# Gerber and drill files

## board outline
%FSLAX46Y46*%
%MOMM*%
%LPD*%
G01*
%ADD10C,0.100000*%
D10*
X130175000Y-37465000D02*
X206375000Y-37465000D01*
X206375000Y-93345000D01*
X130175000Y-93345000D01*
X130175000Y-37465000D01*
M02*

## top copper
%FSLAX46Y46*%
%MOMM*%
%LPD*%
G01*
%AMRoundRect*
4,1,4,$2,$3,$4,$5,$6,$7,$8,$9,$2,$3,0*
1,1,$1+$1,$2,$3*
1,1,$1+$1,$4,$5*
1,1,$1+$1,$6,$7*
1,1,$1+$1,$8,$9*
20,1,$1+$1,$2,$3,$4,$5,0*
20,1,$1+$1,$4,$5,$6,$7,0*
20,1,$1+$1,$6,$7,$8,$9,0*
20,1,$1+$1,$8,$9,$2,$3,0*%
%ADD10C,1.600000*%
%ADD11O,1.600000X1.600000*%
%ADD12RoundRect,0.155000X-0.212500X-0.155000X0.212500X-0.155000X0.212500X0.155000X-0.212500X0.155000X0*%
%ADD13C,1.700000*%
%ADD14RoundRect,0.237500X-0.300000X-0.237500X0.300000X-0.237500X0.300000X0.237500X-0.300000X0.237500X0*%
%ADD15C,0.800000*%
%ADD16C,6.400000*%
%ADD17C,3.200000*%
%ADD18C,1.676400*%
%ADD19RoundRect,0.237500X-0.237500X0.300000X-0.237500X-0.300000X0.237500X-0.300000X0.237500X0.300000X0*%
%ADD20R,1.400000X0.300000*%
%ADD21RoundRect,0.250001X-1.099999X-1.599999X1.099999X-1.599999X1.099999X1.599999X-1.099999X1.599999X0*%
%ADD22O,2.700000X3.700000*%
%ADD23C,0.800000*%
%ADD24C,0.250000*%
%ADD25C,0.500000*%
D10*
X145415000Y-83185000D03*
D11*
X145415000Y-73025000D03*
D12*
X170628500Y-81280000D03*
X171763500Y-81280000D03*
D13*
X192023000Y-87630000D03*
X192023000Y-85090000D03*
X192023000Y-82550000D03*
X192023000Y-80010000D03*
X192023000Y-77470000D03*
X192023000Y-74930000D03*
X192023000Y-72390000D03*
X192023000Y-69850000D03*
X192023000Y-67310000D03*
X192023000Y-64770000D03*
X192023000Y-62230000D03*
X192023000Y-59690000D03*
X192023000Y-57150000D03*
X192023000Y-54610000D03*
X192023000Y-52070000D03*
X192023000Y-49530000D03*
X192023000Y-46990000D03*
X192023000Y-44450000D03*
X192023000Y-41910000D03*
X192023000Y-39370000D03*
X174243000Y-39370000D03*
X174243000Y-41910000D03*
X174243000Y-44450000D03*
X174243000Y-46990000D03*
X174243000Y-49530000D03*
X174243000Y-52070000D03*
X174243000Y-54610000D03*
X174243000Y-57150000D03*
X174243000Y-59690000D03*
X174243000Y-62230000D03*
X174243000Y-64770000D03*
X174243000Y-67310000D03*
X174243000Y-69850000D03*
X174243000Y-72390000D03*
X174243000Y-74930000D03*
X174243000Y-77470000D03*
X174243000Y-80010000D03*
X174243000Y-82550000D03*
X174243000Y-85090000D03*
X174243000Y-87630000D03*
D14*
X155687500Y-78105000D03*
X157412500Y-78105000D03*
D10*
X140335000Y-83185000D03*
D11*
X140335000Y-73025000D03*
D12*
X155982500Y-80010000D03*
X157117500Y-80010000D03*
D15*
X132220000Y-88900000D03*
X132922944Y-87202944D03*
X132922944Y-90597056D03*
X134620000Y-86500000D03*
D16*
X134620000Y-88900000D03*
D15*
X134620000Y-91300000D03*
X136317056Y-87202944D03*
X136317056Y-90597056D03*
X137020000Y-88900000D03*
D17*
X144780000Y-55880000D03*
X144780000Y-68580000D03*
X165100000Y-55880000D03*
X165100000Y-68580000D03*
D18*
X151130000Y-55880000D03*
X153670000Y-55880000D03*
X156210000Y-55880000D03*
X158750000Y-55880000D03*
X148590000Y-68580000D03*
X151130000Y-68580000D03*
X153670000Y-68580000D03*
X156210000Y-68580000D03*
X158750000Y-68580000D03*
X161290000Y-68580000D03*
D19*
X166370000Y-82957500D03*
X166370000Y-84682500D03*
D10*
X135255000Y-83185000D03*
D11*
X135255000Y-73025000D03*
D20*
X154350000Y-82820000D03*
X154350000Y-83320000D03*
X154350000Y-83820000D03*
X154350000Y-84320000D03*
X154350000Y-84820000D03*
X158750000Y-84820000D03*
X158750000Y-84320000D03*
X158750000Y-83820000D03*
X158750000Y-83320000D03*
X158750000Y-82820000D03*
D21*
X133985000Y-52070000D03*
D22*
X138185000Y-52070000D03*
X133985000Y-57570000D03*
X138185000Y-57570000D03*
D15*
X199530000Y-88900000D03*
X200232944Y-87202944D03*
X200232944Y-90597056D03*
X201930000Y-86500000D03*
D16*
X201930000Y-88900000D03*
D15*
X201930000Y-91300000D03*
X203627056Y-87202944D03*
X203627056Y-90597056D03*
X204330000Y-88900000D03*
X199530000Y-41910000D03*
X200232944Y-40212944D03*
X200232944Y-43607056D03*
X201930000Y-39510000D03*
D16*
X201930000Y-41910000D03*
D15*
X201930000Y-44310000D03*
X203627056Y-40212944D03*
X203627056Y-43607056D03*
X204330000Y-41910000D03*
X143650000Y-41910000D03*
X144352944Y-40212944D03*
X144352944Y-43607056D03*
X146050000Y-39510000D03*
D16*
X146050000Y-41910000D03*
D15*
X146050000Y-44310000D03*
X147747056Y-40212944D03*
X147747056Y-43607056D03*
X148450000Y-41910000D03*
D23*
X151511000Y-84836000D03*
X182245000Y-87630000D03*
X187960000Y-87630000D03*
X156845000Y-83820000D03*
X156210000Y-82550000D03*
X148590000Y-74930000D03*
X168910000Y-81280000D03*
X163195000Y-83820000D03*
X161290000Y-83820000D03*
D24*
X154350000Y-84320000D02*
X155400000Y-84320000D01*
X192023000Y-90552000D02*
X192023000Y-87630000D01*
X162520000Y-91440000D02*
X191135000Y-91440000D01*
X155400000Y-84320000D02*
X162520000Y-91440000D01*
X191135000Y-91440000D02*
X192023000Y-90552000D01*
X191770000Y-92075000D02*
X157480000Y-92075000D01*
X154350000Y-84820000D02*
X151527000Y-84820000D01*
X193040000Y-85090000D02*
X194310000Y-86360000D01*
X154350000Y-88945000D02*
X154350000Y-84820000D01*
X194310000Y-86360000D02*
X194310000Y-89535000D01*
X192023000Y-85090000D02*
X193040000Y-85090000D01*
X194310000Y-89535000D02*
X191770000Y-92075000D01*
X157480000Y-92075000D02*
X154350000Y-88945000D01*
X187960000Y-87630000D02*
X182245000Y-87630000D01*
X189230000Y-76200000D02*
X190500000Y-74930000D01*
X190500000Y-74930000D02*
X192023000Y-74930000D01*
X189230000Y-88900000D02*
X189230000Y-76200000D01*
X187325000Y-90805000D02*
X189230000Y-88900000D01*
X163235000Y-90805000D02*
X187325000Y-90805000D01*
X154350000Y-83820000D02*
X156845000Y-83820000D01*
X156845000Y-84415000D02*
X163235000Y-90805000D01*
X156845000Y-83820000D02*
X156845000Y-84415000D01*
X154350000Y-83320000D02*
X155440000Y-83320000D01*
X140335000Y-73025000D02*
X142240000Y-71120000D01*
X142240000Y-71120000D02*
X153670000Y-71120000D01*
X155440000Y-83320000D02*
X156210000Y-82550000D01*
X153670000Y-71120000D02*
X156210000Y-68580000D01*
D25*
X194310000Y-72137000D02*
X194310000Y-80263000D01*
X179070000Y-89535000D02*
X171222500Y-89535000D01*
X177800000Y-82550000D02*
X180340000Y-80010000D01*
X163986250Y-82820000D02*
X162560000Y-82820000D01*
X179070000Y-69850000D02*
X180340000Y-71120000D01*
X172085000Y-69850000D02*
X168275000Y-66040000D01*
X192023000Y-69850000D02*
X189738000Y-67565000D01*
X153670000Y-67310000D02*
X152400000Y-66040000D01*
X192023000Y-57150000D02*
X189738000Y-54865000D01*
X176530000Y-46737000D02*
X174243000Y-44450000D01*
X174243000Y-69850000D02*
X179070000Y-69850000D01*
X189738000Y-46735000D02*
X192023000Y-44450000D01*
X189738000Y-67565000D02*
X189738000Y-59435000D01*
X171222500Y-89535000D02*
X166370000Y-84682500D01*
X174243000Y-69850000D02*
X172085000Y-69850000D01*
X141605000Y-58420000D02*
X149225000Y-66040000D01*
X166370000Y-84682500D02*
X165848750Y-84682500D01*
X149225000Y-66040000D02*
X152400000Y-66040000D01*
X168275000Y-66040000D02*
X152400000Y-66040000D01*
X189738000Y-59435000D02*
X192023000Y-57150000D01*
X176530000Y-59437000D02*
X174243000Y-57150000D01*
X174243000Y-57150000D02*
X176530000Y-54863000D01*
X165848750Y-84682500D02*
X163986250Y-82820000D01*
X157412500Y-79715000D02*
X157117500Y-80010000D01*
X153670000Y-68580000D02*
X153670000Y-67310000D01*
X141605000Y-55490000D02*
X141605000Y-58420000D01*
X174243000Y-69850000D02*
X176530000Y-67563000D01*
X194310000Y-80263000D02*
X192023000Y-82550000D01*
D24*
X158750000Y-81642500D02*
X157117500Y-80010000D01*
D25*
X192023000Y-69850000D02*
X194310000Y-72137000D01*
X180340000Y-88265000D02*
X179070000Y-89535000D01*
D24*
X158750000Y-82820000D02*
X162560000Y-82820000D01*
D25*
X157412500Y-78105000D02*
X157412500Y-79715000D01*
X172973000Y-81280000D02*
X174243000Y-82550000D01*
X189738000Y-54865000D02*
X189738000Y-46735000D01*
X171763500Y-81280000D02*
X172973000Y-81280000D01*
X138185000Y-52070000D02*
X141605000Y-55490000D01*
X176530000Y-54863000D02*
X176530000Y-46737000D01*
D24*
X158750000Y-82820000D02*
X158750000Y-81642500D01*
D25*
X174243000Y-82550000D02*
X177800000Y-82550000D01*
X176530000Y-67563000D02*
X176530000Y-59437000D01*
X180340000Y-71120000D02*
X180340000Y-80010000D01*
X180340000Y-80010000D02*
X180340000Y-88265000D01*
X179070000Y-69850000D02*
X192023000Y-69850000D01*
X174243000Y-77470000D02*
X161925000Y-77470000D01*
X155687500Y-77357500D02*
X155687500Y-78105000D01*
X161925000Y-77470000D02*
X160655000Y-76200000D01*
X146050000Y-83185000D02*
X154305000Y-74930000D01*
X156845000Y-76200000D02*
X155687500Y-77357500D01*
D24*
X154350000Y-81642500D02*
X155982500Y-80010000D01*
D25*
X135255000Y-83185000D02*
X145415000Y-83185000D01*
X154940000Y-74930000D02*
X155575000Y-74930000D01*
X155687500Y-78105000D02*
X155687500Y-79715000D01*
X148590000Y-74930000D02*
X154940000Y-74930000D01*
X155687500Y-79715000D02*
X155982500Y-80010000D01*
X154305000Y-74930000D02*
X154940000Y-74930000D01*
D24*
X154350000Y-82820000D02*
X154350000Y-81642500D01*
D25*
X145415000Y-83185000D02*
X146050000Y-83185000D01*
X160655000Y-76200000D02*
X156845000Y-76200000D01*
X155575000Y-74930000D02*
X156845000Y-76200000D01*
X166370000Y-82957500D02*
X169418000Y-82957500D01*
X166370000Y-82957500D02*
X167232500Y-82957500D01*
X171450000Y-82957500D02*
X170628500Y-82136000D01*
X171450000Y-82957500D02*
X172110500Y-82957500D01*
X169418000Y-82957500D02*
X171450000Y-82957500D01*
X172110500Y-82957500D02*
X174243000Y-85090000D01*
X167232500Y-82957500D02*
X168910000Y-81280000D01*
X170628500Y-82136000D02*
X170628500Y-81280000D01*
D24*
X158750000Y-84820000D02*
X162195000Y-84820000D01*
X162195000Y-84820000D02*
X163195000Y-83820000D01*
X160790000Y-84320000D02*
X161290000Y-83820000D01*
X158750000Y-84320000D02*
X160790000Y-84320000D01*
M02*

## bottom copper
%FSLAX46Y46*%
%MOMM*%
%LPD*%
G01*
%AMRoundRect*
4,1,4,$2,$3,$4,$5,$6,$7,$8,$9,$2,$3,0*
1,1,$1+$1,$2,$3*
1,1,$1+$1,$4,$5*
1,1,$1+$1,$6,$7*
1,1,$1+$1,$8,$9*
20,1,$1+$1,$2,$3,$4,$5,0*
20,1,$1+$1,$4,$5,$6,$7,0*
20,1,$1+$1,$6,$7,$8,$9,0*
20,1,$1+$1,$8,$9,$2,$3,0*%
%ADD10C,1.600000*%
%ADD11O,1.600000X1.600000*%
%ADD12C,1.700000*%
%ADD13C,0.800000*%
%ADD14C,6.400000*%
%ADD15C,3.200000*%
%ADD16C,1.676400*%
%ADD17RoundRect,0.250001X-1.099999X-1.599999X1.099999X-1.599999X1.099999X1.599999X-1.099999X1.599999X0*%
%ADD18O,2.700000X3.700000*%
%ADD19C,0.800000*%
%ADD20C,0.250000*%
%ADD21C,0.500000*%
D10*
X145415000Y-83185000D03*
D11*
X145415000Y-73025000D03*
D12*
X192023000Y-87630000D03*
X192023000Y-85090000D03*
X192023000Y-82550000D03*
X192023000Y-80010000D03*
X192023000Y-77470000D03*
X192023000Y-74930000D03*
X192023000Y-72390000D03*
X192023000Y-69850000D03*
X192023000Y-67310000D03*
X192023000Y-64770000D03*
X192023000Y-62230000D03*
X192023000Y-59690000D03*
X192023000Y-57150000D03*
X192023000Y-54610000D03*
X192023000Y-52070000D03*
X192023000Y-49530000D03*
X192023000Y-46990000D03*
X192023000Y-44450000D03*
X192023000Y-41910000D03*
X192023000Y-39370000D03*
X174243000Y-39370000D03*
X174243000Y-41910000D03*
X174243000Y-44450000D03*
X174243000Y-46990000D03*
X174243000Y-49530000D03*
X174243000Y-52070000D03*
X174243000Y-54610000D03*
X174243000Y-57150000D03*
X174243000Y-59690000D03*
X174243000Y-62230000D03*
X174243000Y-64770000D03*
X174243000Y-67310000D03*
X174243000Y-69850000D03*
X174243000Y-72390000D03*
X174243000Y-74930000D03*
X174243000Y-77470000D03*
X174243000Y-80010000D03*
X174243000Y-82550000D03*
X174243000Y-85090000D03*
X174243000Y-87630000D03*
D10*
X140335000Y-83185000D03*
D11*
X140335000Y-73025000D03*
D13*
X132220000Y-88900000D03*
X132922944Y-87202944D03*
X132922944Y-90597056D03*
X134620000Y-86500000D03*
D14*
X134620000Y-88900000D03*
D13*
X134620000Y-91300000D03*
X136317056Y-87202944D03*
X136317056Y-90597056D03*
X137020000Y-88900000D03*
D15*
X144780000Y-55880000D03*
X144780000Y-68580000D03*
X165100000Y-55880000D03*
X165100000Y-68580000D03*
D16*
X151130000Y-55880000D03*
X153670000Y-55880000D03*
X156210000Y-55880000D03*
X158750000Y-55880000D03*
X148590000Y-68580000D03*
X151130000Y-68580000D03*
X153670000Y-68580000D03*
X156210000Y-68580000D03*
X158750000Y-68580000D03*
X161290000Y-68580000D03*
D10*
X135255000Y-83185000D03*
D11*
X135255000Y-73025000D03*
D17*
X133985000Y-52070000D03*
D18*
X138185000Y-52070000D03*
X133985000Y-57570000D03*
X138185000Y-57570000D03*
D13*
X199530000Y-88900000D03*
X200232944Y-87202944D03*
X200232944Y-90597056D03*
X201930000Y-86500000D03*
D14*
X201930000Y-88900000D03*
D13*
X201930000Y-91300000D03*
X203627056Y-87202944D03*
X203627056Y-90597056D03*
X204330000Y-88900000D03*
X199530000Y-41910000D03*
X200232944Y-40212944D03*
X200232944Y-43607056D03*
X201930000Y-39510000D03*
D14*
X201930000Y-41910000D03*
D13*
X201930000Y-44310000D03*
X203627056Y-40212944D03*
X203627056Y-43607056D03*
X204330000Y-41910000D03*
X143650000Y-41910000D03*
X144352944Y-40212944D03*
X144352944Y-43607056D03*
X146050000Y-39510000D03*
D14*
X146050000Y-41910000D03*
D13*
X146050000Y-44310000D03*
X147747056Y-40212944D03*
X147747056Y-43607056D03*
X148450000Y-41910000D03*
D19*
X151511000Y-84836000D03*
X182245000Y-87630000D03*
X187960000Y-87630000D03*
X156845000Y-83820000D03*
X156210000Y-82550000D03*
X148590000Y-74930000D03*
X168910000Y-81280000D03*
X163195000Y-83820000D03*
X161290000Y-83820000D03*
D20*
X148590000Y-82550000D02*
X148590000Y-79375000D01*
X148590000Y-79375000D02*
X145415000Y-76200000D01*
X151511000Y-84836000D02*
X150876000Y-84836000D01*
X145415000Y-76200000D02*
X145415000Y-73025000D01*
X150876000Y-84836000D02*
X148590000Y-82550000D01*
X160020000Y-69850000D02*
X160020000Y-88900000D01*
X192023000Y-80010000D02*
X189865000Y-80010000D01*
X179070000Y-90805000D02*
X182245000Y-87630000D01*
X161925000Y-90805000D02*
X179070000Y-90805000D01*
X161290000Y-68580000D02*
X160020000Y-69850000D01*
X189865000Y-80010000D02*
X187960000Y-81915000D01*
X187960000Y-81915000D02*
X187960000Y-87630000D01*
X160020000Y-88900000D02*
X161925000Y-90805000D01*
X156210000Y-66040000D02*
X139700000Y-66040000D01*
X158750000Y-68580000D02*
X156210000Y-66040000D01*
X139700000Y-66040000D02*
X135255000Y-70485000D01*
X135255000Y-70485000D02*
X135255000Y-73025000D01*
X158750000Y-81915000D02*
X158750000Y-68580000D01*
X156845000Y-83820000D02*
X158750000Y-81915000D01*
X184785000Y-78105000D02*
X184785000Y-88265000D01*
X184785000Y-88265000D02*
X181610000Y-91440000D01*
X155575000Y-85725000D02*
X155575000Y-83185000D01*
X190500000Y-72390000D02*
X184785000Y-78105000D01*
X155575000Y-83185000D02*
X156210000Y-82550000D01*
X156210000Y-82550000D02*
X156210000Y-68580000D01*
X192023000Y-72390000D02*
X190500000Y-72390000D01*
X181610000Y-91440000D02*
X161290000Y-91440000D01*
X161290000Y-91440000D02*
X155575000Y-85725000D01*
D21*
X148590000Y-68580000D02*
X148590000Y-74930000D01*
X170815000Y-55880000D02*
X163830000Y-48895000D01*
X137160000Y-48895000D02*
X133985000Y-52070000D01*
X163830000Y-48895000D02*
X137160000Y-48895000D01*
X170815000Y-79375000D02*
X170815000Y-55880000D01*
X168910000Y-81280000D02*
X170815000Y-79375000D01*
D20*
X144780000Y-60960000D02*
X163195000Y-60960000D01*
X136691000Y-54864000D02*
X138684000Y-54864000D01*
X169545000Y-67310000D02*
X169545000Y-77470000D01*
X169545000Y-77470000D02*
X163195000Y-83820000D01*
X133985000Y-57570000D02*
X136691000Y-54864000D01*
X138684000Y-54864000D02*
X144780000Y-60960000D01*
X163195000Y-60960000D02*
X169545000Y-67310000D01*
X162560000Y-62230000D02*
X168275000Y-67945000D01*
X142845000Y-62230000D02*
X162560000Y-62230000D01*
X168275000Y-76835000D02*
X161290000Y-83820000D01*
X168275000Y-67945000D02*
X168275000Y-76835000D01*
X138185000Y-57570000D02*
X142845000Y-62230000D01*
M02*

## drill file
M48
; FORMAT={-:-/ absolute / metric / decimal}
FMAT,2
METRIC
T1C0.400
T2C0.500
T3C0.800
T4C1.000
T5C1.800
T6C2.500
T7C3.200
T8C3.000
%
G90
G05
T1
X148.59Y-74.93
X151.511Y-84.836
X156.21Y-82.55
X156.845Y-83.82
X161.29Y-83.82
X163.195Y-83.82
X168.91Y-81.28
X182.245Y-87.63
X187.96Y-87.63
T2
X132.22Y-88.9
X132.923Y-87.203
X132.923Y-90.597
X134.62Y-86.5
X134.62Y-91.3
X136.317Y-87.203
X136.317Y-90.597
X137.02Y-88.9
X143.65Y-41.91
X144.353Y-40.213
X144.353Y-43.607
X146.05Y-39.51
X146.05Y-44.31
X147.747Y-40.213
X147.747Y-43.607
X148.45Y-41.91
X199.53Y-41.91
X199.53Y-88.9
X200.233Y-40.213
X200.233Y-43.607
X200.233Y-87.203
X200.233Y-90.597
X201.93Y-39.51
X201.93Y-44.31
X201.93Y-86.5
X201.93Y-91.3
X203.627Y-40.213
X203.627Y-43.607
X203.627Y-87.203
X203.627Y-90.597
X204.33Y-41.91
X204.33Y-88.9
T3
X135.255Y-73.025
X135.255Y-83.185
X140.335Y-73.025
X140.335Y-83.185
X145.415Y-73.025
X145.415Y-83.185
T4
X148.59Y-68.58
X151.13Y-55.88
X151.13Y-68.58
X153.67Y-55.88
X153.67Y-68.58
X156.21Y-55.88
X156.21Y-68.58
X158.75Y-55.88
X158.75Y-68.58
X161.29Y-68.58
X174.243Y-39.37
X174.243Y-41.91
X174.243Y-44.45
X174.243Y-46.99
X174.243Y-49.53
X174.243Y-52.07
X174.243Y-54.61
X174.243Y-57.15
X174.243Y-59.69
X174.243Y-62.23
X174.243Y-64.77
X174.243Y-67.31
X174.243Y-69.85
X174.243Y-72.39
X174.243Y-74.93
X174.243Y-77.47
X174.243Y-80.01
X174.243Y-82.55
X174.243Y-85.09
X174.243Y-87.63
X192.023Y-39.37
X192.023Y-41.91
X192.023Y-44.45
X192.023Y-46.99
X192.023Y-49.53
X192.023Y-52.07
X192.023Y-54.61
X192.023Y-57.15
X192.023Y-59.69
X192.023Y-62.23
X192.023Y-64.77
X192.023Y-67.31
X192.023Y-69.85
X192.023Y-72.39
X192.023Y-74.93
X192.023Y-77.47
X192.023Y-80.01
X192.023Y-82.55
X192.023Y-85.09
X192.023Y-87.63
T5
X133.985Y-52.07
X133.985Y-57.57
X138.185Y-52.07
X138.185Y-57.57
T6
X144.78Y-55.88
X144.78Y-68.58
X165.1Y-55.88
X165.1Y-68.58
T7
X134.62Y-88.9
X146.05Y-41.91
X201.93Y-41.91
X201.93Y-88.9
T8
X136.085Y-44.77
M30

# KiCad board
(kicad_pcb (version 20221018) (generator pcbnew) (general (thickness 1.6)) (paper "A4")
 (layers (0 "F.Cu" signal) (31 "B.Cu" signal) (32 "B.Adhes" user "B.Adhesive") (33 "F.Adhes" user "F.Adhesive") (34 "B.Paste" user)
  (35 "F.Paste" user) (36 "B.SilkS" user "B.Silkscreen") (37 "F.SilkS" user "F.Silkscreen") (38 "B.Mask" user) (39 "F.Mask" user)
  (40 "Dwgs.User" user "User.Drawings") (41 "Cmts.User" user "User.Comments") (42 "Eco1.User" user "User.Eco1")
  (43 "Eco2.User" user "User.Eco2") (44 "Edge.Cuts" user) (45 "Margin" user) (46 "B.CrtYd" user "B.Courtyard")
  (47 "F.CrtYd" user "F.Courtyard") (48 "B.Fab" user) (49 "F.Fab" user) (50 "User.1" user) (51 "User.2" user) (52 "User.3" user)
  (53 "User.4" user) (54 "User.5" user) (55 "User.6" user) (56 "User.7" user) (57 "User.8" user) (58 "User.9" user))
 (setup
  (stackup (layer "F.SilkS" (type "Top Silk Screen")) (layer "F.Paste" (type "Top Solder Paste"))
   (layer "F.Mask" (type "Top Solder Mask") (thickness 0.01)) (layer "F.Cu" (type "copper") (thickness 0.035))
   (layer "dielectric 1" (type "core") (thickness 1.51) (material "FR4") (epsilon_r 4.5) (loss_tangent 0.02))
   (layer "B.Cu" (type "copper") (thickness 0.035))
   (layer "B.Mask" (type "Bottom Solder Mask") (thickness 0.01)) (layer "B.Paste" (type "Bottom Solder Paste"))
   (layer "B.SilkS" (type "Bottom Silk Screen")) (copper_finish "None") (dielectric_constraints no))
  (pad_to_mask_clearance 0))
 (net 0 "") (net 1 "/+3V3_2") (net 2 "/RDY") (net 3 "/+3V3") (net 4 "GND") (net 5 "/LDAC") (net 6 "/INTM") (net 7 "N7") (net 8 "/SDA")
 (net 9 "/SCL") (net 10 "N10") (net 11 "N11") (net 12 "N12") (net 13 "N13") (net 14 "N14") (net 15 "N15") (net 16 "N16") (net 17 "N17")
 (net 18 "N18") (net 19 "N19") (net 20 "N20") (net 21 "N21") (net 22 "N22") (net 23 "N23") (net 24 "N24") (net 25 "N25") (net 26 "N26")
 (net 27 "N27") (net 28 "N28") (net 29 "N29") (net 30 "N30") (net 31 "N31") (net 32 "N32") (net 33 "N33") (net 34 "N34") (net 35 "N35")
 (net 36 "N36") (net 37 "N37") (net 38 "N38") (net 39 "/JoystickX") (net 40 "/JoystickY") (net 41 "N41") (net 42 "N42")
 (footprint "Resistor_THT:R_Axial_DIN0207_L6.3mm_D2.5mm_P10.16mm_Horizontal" (layer "F.Cu") (at 145.415 83.185 90)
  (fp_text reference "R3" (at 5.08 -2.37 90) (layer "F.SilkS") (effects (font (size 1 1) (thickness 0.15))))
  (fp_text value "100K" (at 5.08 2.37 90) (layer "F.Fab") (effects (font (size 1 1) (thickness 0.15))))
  (pad "1" thru_hole circle (at 0 0 90) (size 1.6 1.6) (drill 0.8) (layers "*.Cu" "*.Mask") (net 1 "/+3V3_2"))
  (pad "2" thru_hole oval (at 10.16 0 90) (size 1.6 1.6) (drill 0.8) (layers "*.Cu" "*.Mask") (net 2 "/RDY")))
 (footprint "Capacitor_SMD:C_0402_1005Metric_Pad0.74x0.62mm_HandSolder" (layer "F.Cu") (at 171.196 81.28)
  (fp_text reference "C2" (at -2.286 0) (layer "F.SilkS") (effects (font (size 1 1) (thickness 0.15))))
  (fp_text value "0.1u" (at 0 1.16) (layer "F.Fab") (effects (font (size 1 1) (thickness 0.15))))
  (pad "1" smd roundrect (at -0.5675 0) (size 0.735 0.62) (layers "F.Cu" "F.Paste" "F.Mask") (roundrect_rratio 0.25) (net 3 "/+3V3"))
  (pad "2" smd roundrect (at 0.5675 0) (size 0.735 0.62) (layers "F.Cu" "F.Paste" "F.Mask") (roundrect_rratio 0.25) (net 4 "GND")))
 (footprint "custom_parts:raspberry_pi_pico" (layer "F.Cu") (at 183.515 64.712 90)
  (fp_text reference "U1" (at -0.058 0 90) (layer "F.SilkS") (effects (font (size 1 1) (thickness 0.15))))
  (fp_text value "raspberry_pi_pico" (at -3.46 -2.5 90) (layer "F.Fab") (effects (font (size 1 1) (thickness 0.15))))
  (pad "1" thru_hole circle (at -22.918 8.508) (size 1.7 1.7) (drill 1) (layers "*.Cu" "*.Mask") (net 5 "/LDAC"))
  (pad "2" thru_hole circle (at -20.378 8.508) (size 1.7 1.7) (drill 1) (layers "*.Cu" "*.Mask") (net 2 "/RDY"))
  (pad "3" thru_hole circle (at -17.838 8.508) (size 1.7 1.7) (drill 1) (layers "*.Cu" "*.Mask") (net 4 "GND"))
  (pad "4" thru_hole circle (at -15.298 8.508) (size 1.7 1.7) (drill 1) (layers "*.Cu" "*.Mask") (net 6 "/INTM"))
  (pad "5" thru_hole circle (at -12.758 8.508) (size 1.7 1.7) (drill 1) (layers "*.Cu" "*.Mask") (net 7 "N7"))
  (pad "6" thru_hole circle (at -10.218 8.508) (size 1.7 1.7) (drill 1) (layers "*.Cu" "*.Mask") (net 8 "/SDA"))
  (pad "7" thru_hole circle (at -7.678 8.508) (size 1.7 1.7) (drill 1) (layers "*.Cu" "*.Mask") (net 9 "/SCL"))
  (pad "8" thru_hole circle (at -5.138 8.508) (size 1.7 1.7) (drill 1) (layers "*.Cu" "*.Mask") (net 4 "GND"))
  (pad "9" thru_hole circle (at -2.598 8.508) (size 1.7 1.7) (drill 1) (layers "*.Cu" "*.Mask") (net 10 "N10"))
  (pad "10" thru_hole circle (at -0.058 8.508) (size 1.7 1.7) (drill 1) (layers "*.Cu" "*.Mask") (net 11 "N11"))
  (pad "11" thru_hole circle (at 2.482 8.508) (size 1.7 1.7) (drill 1) (layers "*.Cu" "*.Mask") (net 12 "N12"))
  (pad "12" thru_hole circle (at 5.022 8.508) (size 1.7 1.7) (drill 1) (layers "*.Cu" "*.Mask") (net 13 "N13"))
  (pad "13" thru_hole circle (at 7.562 8.508) (size 1.7 1.7) (drill 1) (layers "*.Cu" "*.Mask") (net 4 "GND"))
  (pad "14" thru_hole circle (at 10.102 8.508) (size 1.7 1.7) (drill 1) (layers "*.Cu" "*.Mask") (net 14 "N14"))
  (pad "15" thru_hole circle (at 12.642 8.508) (size 1.7 1.7) (drill 1) (layers "*.Cu" "*.Mask") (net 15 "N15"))
  (pad "16" thru_hole circle (at 15.182 8.508) (size 1.7 1.7) (drill 1) (layers "*.Cu" "*.Mask") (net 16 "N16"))
  (pad "17" thru_hole circle (at 17.722 8.508) (size 1.7 1.7) (drill 1) (layers "*.Cu" "*.Mask") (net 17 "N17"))
  (pad "18" thru_hole circle (at 20.262 8.508) (size 1.7 1.7) (drill 1) (layers "*.Cu" "*.Mask") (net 4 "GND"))
  (pad "19" thru_hole circle (at 22.802 8.508) (size 1.7 1.7) (drill 1) (layers "*.Cu" "*.Mask") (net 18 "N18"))
  (pad "20" thru_hole circle (at 25.342 8.508) (size 1.7 1.7) (drill 1) (layers "*.Cu" "*.Mask") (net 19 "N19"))
  (pad "21" thru_hole circle (at 25.342 -9.272) (size 1.7 1.7) (drill 1) (layers "*.Cu" "*.Mask") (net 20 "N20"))
  (pad "22" thru_hole circle (at 22.802 -9.272) (size 1.7 1.7) (drill 1) (layers "*.Cu" "*.Mask") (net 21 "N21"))
  (pad "23" thru_hole circle (at 20.262 -9.272) (size 1.7 1.7) (drill 1) (layers "*.Cu" "*.Mask") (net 4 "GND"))
  (pad "24" thru_hole circle (at 17.722 -9.272) (size 1.7 1.7) (drill 1) (layers "*.Cu" "*.Mask") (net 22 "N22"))
  (pad "25" thru_hole circle (at 15.182 -9.272) (size 1.7 1.7) (drill 1) (layers "*.Cu" "*.Mask") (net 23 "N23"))
  (pad "26" thru_hole circle (at 12.642 -9.272) (size 1.7 1.7) (drill 1) (layers "*.Cu" "*.Mask") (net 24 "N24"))
  (pad "27" thru_hole circle (at 10.102 -9.272) (size 1.7 1.7) (drill 1) (layers "*.Cu" "*.Mask") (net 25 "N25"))
  (pad "28" thru_hole circle (at 7.562 -9.272) (size 1.7 1.7) (drill 1) (layers "*.Cu" "*.Mask") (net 4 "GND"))
  (pad "29" thru_hole circle (at 5.022 -9.272) (size 1.7 1.7) (drill 1) (layers "*.Cu" "*.Mask") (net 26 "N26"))
  (pad "30" thru_hole circle (at 2.482 -9.272) (size 1.7 1.7) (drill 1) (layers "*.Cu" "*.Mask") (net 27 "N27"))
  (pad "31" thru_hole circle (at -0.058 -9.272) (size 1.7 1.7) (drill 1) (layers "*.Cu" "*.Mask") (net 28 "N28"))
  (pad "32" thru_hole circle (at -2.598 -9.272) (size 1.7 1.7) (drill 1) (layers "*.Cu" "*.Mask") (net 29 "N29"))
  (pad "33" thru_hole circle (at -5.138 -9.272) (size 1.7 1.7) (drill 1) (layers "*.Cu" "*.Mask") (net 4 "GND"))
  (pad "34" thru_hole circle (at -7.678 -9.272) (size 1.7 1.7) (drill 1) (layers "*.Cu" "*.Mask") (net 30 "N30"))
  (pad "35" thru_hole circle (at -10.218 -9.272) (size 1.7 1.7) (drill 1) (layers "*.Cu" "*.Mask") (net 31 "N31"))
  (pad "36" thru_hole circle (at -12.758 -9.272) (size 1.7 1.7) (drill 1) (layers "*.Cu" "*.Mask") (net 1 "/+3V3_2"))
  (pad "37" thru_hole circle (at -15.298 -9.272) (size 1.7 1.7) (drill 1) (layers "*.Cu" "*.Mask") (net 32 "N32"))
  (pad "38" thru_hole circle (at -17.838 -9.272) (size 1.7 1.7) (drill 1) (layers "*.Cu" "*.Mask") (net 4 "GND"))
  (pad "39" thru_hole circle (at -20.378 -9.272) (size 1.7 1.7) (drill 1) (layers "*.Cu" "*.Mask") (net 3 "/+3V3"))
  (pad "40" thru_hole circle (at -22.918 -9.272) (size 1.7 1.7) (drill 1) (layers "*.Cu" "*.Mask") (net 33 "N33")))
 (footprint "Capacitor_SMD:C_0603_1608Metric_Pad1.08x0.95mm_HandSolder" (layer "F.Cu") (at 156.55 78.105)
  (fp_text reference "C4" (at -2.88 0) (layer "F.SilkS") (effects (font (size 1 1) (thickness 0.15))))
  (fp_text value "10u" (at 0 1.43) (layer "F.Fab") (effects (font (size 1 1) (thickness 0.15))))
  (pad "1" smd roundrect (at -0.8625 0) (size 1.075 0.95) (layers "F.Cu" "F.Paste" "F.Mask") (roundrect_rratio 0.25) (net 1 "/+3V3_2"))
  (pad "2" smd roundrect (at 0.8625 0) (size 1.075 0.95) (layers "F.Cu" "F.Paste" "F.Mask") (roundrect_rratio 0.25) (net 4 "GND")))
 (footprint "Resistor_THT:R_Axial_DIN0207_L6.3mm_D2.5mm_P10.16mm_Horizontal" (layer "F.Cu") (at 140.335 83.185 90)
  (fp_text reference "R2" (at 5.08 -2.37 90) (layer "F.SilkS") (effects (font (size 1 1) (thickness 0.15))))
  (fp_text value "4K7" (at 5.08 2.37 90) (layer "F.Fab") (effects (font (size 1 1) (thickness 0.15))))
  (pad "1" thru_hole circle (at 0 0 90) (size 1.6 1.6) (drill 0.8) (layers "*.Cu" "*.Mask") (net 1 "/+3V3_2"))
  (pad "2" thru_hole oval (at 10.16 0 90) (size 1.6 1.6) (drill 0.8) (layers "*.Cu" "*.Mask") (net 9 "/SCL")))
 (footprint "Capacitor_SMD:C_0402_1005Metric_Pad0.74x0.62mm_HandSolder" (layer "F.Cu") (at 156.55 80.01)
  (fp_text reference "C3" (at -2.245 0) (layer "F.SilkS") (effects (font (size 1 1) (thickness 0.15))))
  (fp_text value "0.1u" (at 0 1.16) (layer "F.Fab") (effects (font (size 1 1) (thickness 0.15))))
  (pad "1" smd roundrect (at -0.5675 0) (size 0.735 0.62) (layers "F.Cu" "F.Paste" "F.Mask") (roundrect_rratio 0.25) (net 1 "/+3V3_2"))
  (pad "2" smd roundrect (at 0.5675 0) (size 0.735 0.62) (layers "F.Cu" "F.Paste" "F.Mask") (roundrect_rratio 0.25) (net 4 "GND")))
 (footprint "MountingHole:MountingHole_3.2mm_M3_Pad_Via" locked (layer "F.Cu") (at 134.62 88.9)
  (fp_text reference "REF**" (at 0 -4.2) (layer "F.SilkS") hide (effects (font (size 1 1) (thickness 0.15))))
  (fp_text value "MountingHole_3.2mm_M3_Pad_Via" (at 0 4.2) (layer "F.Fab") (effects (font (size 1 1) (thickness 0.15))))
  (pad "1" thru_hole circle locked (at -2.4 0) (size 0.8 0.8) (drill 0.5) (layers "*.Cu" "*.Mask"))
  (pad "1" thru_hole circle locked (at -1.697056 -1.697056) (size 0.8 0.8) (drill 0.5) (layers "*.Cu" "*.Mask"))
  (pad "1" thru_hole circle locked (at -1.697056 1.697056) (size 0.8 0.8) (drill 0.5) (layers "*.Cu" "*.Mask"))
  (pad "1" thru_hole circle locked (at 0 -2.4) (size 0.8 0.8) (drill 0.5) (layers "*.Cu" "*.Mask"))
  (pad "1" thru_hole circle locked (at 0 0) (size 6.4 6.4) (drill 3.2) (layers "*.Cu" "*.Mask"))
  (pad "1" thru_hole circle locked (at 0 2.4) (size 0.8 0.8) (drill 0.5) (layers "*.Cu" "*.Mask"))
  (pad "1" thru_hole circle locked (at 1.697056 -1.697056) (size 0.8 0.8) (drill 0.5) (layers "*.Cu" "*.Mask"))
  (pad "1" thru_hole circle locked (at 1.697056 1.697056) (size 0.8 0.8) (drill 0.5) (layers "*.Cu" "*.Mask"))
  (pad "1" thru_hole circle locked (at 2.4 0) (size 0.8 0.8) (drill 0.5) (layers "*.Cu" "*.Mask")))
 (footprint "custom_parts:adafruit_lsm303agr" (layer "F.Cu") (at 154.94 63.5)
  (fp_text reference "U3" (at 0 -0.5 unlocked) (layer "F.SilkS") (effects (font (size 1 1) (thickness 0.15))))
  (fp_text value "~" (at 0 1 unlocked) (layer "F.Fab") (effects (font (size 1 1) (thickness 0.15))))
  (pad "" thru_hole circle (at -10.16 -7.62) (size 3.2 3.2) (drill 2.5) (layers "*.Cu" "*.Mask") (zone_connect 0))
  (pad "" thru_hole circle (at -10.16 5.08) (size 3.2 3.2) (drill 2.5) (layers "*.Cu" "*.Mask") (zone_connect 0))
  (pad "" thru_hole circle (at 10.16 -7.62) (size 3.2 3.2) (drill 2.5) (layers "*.Cu" "*.Mask") (zone_connect 0))
  (pad "" thru_hole circle (at 10.16 5.08) (size 3.2 3.2) (drill 2.5) (layers "*.Cu" "*.Mask") (zone_connect 0))
  (pad "0" thru_hole circle (at -3.81 -7.62 90) (size 1.6764 1.6764) (drill 1) (layers "*.Cu" "*.Mask") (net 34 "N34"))
  (pad "1" thru_hole circle (at -1.27 -7.62 90) (size 1.6764 1.6764) (drill 1) (layers "*.Cu" "*.Mask") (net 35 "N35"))
  (pad "2" thru_hole circle (at 1.27 -7.62 90) (size 1.6764 1.6764) (drill 1) (layers "*.Cu" "*.Mask") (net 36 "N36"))
  (pad "3" thru_hole circle (at 3.81 -7.62 90) (size 1.6764 1.6764) (drill 1) (layers "*.Cu" "*.Mask") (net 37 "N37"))
  (pad "4" thru_hole circle (at -6.35 5.08 90) (size 1.6764 1.6764) (drill 1) (layers "*.Cu" "*.Mask") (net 1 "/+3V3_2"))
  (pad "5" thru_hole circle (at -3.81 5.08 90) (size 1.6764 1.6764) (drill 1) (layers "*.Cu" "*.Mask") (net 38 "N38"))
  (pad "6" thru_hole circle (at -1.27 5.08 90) (size 1.6764 1.6764) (drill 1) (layers "*.Cu" "*.Mask") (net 4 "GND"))
  (pad "7" thru_hole circle (at 1.27 5.08 90) (size 1.6764 1.6764) (drill 1) (layers "*.Cu" "*.Mask") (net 9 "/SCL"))
  (pad "8" thru_hole circle (at 3.81 5.08 90) (size 1.6764 1.6764) (drill 1) (layers "*.Cu" "*.Mask") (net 8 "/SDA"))
  (pad "9" thru_hole circle (at 6.35 5.08 90) (size 1.6764 1.6764) (drill 1) (layers "*.Cu" "*.Mask") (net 6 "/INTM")))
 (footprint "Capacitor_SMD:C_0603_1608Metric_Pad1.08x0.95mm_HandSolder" (layer "F.Cu") (at 166.37 83.82 -90)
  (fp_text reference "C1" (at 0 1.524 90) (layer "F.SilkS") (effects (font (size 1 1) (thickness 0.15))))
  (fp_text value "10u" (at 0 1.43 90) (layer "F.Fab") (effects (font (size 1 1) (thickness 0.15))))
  (pad "1" smd roundrect (at -0.8625 0 270) (size 1.075 0.95) (layers "F.Cu" "F.Paste" "F.Mask") (roundrect_rratio 0.25) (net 3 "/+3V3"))
  (pad "2" smd roundrect (at 0.8625 0 270) (size 1.075 0.95) (layers "F.Cu" "F.Paste" "F.Mask") (roundrect_rratio 0.25) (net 4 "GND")))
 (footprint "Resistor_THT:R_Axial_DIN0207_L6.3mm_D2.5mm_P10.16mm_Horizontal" (layer "F.Cu") (at 135.255 83.185 90)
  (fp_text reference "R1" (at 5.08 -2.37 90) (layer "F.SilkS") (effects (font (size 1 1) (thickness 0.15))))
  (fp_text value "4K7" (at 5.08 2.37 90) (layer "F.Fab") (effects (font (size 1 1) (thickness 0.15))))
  (pad "1" thru_hole circle (at 0 0 90) (size 1.6 1.6) (drill 0.8) (layers "*.Cu" "*.Mask") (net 1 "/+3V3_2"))
  (pad "2" thru_hole oval (at 10.16 0 90) (size 1.6 1.6) (drill 0.8) (layers "*.Cu" "*.Mask") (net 8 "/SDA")))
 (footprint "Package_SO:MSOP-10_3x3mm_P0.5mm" (layer "F.Cu") (at 156.55 83.82)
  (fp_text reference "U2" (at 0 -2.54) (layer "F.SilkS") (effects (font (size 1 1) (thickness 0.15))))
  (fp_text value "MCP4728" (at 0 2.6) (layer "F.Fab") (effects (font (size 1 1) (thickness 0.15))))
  (pad "1" smd rect (at -2.2 -1) (size 1.4 0.3) (layers "F.Cu" "F.Paste" "F.Mask") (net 1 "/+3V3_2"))
  (pad "2" smd rect (at -2.2 -0.5) (size 1.4 0.3) (layers "F.Cu" "F.Paste" "F.Mask") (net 9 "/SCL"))
  (pad "3" smd rect (at -2.2 0) (size 1.4 0.3) (layers "F.Cu" "F.Paste" "F.Mask") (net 8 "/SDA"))
  (pad "4" smd rect (at -2.2 0.5) (size 1.4 0.3) (layers "F.Cu" "F.Paste" "F.Mask") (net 5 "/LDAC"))
  (pad "5" smd rect (at -2.2 1) (size 1.4 0.3) (layers "F.Cu" "F.Paste" "F.Mask") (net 2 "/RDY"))
  (pad "6" smd rect (at 2.2 1) (size 1.4 0.3) (layers "F.Cu" "F.Paste" "F.Mask") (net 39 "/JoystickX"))
  (pad "7" smd rect (at 2.2 0.5) (size 1.4 0.3) (layers "F.Cu" "F.Paste" "F.Mask") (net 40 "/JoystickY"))
  (pad "8" smd rect (at 2.2 0) (size 1.4 0.3) (layers "F.Cu" "F.Paste" "F.Mask") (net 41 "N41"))
  (pad "9" smd rect (at 2.2 -0.5) (size 1.4 0.3) (layers "F.Cu" "F.Paste" "F.Mask") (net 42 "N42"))
  (pad "10" smd rect (at 2.2 -1) (size 1.4 0.3) (layers "F.Cu" "F.Paste" "F.Mask") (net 4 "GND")))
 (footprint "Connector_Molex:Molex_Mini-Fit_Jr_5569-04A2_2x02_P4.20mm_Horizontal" (layer "F.Cu") (at 133.985 52.07)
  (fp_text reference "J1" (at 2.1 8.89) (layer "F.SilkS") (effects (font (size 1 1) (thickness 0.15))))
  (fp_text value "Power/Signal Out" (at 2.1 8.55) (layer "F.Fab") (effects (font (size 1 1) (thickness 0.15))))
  (pad "" np_thru_hole circle (at 2.1 -7.3) (size 3 3) (drill 3) (layers "*.Cu" "*.Mask"))
  (pad "1" thru_hole roundrect (at 0 0) (size 2.7 3.7) (drill 1.8) (layers "*.Cu" "*.Mask") (roundrect_rratio 0.09259296296) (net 3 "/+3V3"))
  (pad "2" thru_hole oval (at 4.2 0) (size 2.7 3.7) (drill 1.8) (layers "*.Cu" "*.Mask") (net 4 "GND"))
  (pad "3" thru_hole oval (at 0 5.5) (size 2.7 3.7) (drill 1.8) (layers "*.Cu" "*.Mask") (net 39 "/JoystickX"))
  (pad "4" thru_hole oval (at 4.2 5.5) (size 2.7 3.7) (drill 1.8) (layers "*.Cu" "*.Mask") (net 40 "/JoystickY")))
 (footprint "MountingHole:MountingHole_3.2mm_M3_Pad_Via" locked (layer "F.Cu") (at 201.93 88.9)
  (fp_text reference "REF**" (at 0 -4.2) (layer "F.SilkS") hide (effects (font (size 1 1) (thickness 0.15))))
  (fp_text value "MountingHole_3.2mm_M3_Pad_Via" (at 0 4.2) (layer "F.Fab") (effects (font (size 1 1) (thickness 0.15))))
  (pad "1" thru_hole circle locked (at -2.4 0) (size 0.8 0.8) (drill 0.5) (layers "*.Cu" "*.Mask"))
  (pad "1" thru_hole circle locked (at -1.697056 -1.697056) (size 0.8 0.8) (drill 0.5) (layers "*.Cu" "*.Mask"))
  (pad "1" thru_hole circle locked (at -1.697056 1.697056) (size 0.8 0.8) (drill 0.5) (layers "*.Cu" "*.Mask"))
  (pad "1" thru_hole circle locked (at 0 -2.4) (size 0.8 0.8) (drill 0.5) (layers "*.Cu" "*.Mask"))
  (pad "1" thru_hole circle locked (at 0 0) (size 6.4 6.4) (drill 3.2) (layers "*.Cu" "*.Mask"))
  (pad "1" thru_hole circle locked (at 0 2.4) (size 0.8 0.8) (drill 0.5) (layers "*.Cu" "*.Mask"))
  (pad "1" thru_hole circle locked (at 1.697056 -1.697056) (size 0.8 0.8) (drill 0.5) (layers "*.Cu" "*.Mask"))
  (pad "1" thru_hole circle locked (at 1.697056 1.697056) (size 0.8 0.8) (drill 0.5) (layers "*.Cu" "*.Mask"))
  (pad "1" thru_hole circle locked (at 2.4 0) (size 0.8 0.8) (drill 0.5) (layers "*.Cu" "*.Mask")))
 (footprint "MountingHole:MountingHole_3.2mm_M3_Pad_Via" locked (layer "F.Cu") (at 201.93 41.91)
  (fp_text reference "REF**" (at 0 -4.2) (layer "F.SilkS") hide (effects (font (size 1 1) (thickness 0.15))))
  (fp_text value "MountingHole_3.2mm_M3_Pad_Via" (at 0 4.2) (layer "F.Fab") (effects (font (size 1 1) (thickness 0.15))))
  (pad "1" thru_hole circle locked (at -2.4 0) (size 0.8 0.8) (drill 0.5) (layers "*.Cu" "*.Mask"))
  (pad "1" thru_hole circle locked (at -1.697056 -1.697056) (size 0.8 0.8) (drill 0.5) (layers "*.Cu" "*.Mask"))
  (pad "1" thru_hole circle locked (at -1.697056 1.697056) (size 0.8 0.8) (drill 0.5) (layers "*.Cu" "*.Mask"))
  (pad "1" thru_hole circle locked (at 0 -2.4) (size 0.8 0.8) (drill 0.5) (layers "*.Cu" "*.Mask"))
  (pad "1" thru_hole circle locked (at 0 0) (size 6.4 6.4) (drill 3.2) (layers "*.Cu" "*.Mask"))
  (pad "1" thru_hole circle locked (at 0 2.4) (size 0.8 0.8) (drill 0.5) (layers "*.Cu" "*.Mask"))
  (pad "1" thru_hole circle locked (at 1.697056 -1.697056) (size 0.8 0.8) (drill 0.5) (layers "*.Cu" "*.Mask"))
  (pad "1" thru_hole circle locked (at 1.697056 1.697056) (size 0.8 0.8) (drill 0.5) (layers "*.Cu" "*.Mask"))
  (pad "1" thru_hole circle locked (at 2.4 0) (size 0.8 0.8) (drill 0.5) (layers "*.Cu" "*.Mask")))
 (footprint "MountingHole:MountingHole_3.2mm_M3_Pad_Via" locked (layer "F.Cu") (at 146.05 41.91)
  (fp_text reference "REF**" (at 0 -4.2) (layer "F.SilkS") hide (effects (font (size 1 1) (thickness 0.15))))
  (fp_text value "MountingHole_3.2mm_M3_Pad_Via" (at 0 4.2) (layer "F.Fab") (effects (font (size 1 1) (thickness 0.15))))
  (pad "1" thru_hole circle locked (at -2.4 0) (size 0.8 0.8) (drill 0.5) (layers "*.Cu" "*.Mask"))
  (pad "1" thru_hole circle locked (at -1.697056 -1.697056) (size 0.8 0.8) (drill 0.5) (layers "*.Cu" "*.Mask"))
  (pad "1" thru_hole circle locked (at -1.697056 1.697056) (size 0.8 0.8) (drill 0.5) (layers "*.Cu" "*.Mask"))
  (pad "1" thru_hole circle locked (at 0 -2.4) (size 0.8 0.8) (drill 0.5) (layers "*.Cu" "*.Mask"))
  (pad "1" thru_hole circle locked (at 0 0) (size 6.4 6.4) (drill 3.2) (layers "*.Cu" "*.Mask"))
  (pad "1" thru_hole circle locked (at 0 2.4) (size 0.8 0.8) (drill 0.5) (layers "*.Cu" "*.Mask"))
  (pad "1" thru_hole circle locked (at 1.697056 -1.697056) (size 0.8 0.8) (drill 0.5) (layers "*.Cu" "*.Mask"))
  (pad "1" thru_hole circle locked (at 1.697056 1.697056) (size 0.8 0.8) (drill 0.5) (layers "*.Cu" "*.Mask"))
  (pad "1" thru_hole circle locked (at 2.4 0) (size 0.8 0.8) (drill 0.5) (layers "*.Cu" "*.Mask")))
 (gr_rect (start 130.175 37.465) (end 206.375 93.345) (stroke (width 0.1) (type default)) (fill none) (layer "Edge.Cuts"))
 (segment (start 154.35 84.32) (end 155.4 84.32) (width 0.25) (layer "F.Cu") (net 5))
 (segment (start 192.023 90.552) (end 192.023 87.63) (width 0.25) (layer "F.Cu") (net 5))
 (segment (start 162.52 91.44) (end 191.135 91.44) (width 0.25) (layer "F.Cu") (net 5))
 (segment (start 155.4 84.32) (end 162.52 91.44) (width 0.25) (layer "F.Cu") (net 5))
 (segment (start 191.135 91.44) (end 192.023 90.552) (width 0.25) (layer "F.Cu") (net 5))
 (segment (start 191.77 92.075) (end 157.48 92.075) (width 0.25) (layer "F.Cu") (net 2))
 (segment (start 154.35 84.82) (end 151.527 84.82) (width 0.25) (layer "F.Cu") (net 2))
 (segment (start 193.04 85.09) (end 194.31 86.36) (width 0.25) (layer "F.Cu") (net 2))
 (segment (start 154.35 88.945) (end 154.35 84.82) (width 0.25) (layer "F.Cu") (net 2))
 (segment (start 194.31 86.36) (end 194.31 89.535) (width 0.25) (layer "F.Cu") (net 2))
 (segment (start 192.023 85.09) (end 193.04 85.09) (width 0.25) (layer "F.Cu") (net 2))
 (segment (start 194.31 89.535) (end 191.77 92.075) (width 0.25) (layer "F.Cu") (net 2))
 (segment (start 157.48 92.075) (end 154.35 88.945) (width 0.25) (layer "F.Cu") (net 2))
 (via (at 151.511 84.836) (size 0.8) (drill 0.4) (layers "F.Cu" "B.Cu") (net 2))
 (segment (start 148.59 82.55) (end 148.59 79.375) (width 0.25) (layer "B.Cu") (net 2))
 (segment (start 148.59 79.375) (end 145.415 76.2) (width 0.25) (layer "B.Cu") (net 2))
 (segment (start 151.511 84.836) (end 150.876 84.836) (width 0.25) (layer "B.Cu") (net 2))
 (segment (start 145.415 76.2) (end 145.415 73.025) (width 0.25) (layer "B.Cu") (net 2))
 (segment (start 150.876 84.836) (end 148.59 82.55) (width 0.25) (layer "B.Cu") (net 2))
 (segment (start 187.96 87.63) (end 182.245 87.63) (width 0.25) (layer "F.Cu") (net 6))
 (via (at 182.245 87.63) (size 0.8) (drill 0.4) (layers "F.Cu" "B.Cu") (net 6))
 (via (at 187.96 87.63) (size 0.8) (drill 0.4) (layers "F.Cu" "B.Cu") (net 6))
 (segment (start 160.02 69.85) (end 160.02 88.9) (width 0.25) (layer "B.Cu") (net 6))
 (segment (start 192.023 80.01) (end 189.865 80.01) (width 0.25) (layer "B.Cu") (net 6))
 (segment (start 179.07 90.805) (end 182.245 87.63) (width 0.25) (layer "B.Cu") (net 6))
 (segment (start 161.925 90.805) (end 179.07 90.805) (width 0.25) (layer "B.Cu") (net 6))
 (segment (start 161.29 68.58) (end 160.02 69.85) (width 0.25) (layer "B.Cu") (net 6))
 (segment (start 189.865 80.01) (end 187.96 81.915) (width 0.25) (layer "B.Cu") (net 6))
 (segment (start 187.96 81.915) (end 187.96 87.63) (width 0.25) (layer "B.Cu") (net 6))
 (segment (start 160.02 88.9) (end 161.925 90.805) (width 0.25) (layer "B.Cu") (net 6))
 (segment (start 189.23 76.2) (end 190.5 74.93) (width 0.25) (layer "F.Cu") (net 8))
 (segment (start 190.5 74.93) (end 192.023 74.93) (width 0.25) (layer "F.Cu") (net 8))
 (segment (start 189.23 88.9) (end 189.23 76.2) (width 0.25) (layer "F.Cu") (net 8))
 (segment (start 187.325 90.805) (end 189.23 88.9) (width 0.25) (layer "F.Cu") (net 8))
 (segment (start 163.235 90.805) (end 187.325 90.805) (width 0.25) (layer "F.Cu") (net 8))
 (segment (start 154.35 83.82) (end 156.845 83.82) (width 0.25) (layer "F.Cu") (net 8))
 (segment (start 156.845 84.415) (end 163.235 90.805) (width 0.25) (layer "F.Cu") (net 8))
 (segment (start 156.845 83.82) (end 156.845 84.415) (width 0.25) (layer "F.Cu") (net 8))
 (via (at 156.845 83.82) (size 0.8) (drill 0.4) (layers "F.Cu" "B.Cu") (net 8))
 (segment (start 156.21 66.04) (end 139.7 66.04) (width 0.25) (layer "B.Cu") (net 8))
 (segment (start 158.75 68.58) (end 156.21 66.04) (width 0.25) (layer "B.Cu") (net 8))
 (segment (start 139.7 66.04) (end 135.255 70.485) (width 0.25) (layer "B.Cu") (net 8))
 (segment (start 135.255 70.485) (end 135.255 73.025) (width 0.25) (layer "B.Cu") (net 8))
 (segment (start 158.75 81.915) (end 158.75 68.58) (width 0.25) (layer "B.Cu") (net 8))
 (segment (start 156.845 83.82) (end 158.75 81.915) (width 0.25) (layer "B.Cu") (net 8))
 (segment (start 154.35 83.32) (end 155.44 83.32) (width 0.25) (layer "F.Cu") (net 9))
 (segment (start 140.335 73.025) (end 142.24 71.12) (width 0.25) (layer "F.Cu") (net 9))
 (segment (start 142.24 71.12) (end 153.67 71.12) (width 0.25) (layer "F.Cu") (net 9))
 (segment (start 155.44 83.32) (end 156.21 82.55) (width 0.25) (layer "F.Cu") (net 9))
 (segment (start 153.67 71.12) (end 156.21 68.58) (width 0.25) (layer "F.Cu") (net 9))
 (via (at 156.21 82.55) (size 0.8) (drill 0.4) (layers "F.Cu" "B.Cu") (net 9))
 (segment (start 184.785 78.105) (end 184.785 88.265) (width 0.25) (layer "B.Cu") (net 9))
 (segment (start 184.785 88.265) (end 181.61 91.44) (width 0.25) (layer "B.Cu") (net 9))
 (segment (start 155.575 85.725) (end 155.575 83.185) (width 0.25) (layer "B.Cu") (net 9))
 (segment (start 190.5 72.39) (end 184.785 78.105) (width 0.25) (layer "B.Cu") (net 9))
 (segment (start 155.575 83.185) (end 156.21 82.55) (width 0.25) (layer "B.Cu") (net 9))
 (segment (start 156.21 82.55) (end 156.21 68.58) (width 0.25) (layer "B.Cu") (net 9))
 (segment (start 192.023 72.39) (end 190.5 72.39) (width 0.25) (layer "B.Cu") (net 9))
 (segment (start 181.61 91.44) (end 161.29 91.44) (width 0.25) (layer "B.Cu") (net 9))
 (segment (start 161.29 91.44) (end 155.575 85.725) (width 0.25) (layer "B.Cu") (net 9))
 (segment (start 194.31 72.137) (end 194.31 80.263) (width 0.5) (layer "F.Cu") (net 4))
 (segment (start 179.07 89.535) (end 171.2225 89.535) (width 0.5) (layer "F.Cu") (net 4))
 (segment (start 177.8 82.55) (end 180.34 80.01) (width 0.5) (layer "F.Cu") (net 4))
 (segment (start 163.98625 82.82) (end 162.56 82.82) (width 0.5) (layer "F.Cu") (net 4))
 (segment (start 179.07 69.85) (end 180.34 71.12) (width 0.5) (layer "F.Cu") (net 4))
 (segment (start 172.085 69.85) (end 168.275 66.04) (width 0.5) (layer "F.Cu") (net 4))
 (segment (start 192.023 69.85) (end 189.738 67.565) (width 0.5) (layer "F.Cu") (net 4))
 (segment (start 153.67 67.31) (end 152.4 66.04) (width 0.5) (layer "F.Cu") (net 4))
 (segment (start 192.023 57.15) (end 189.738 54.865) (width 0.5) (layer "F.Cu") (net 4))
 (segment (start 176.53 46.737) (end 174.243 44.45) (width 0.5) (layer "F.Cu") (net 4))
 (segment (start 174.243 69.85) (end 179.07 69.85) (width 0.5) (layer "F.Cu") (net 4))
 (segment (start 189.738 46.735) (end 192.023 44.45) (width 0.5) (layer "F.Cu") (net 4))
 (segment (start 189.738 67.565) (end 189.738 59.435) (width 0.5) (layer "F.Cu") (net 4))
 (segment (start 171.2225 89.535) (end 166.37 84.6825) (width 0.5) (layer "F.Cu") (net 4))
 (segment (start 174.243 69.85) (end 172.085 69.85) (width 0.5) (layer "F.Cu") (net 4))
 (segment (start 141.605 58.42) (end 149.225 66.04) (width 0.5) (layer "F.Cu") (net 4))
 (segment (start 166.37 84.6825) (end 165.84875 84.6825) (width 0.5) (layer "F.Cu") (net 4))
 (segment (start 149.225 66.04) (end 152.4 66.04) (width 0.5) (layer "F.Cu") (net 4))
 (segment (start 168.275 66.04) (end 152.4 66.04) (width 0.5) (layer "F.Cu") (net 4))
 (segment (start 189.738 59.435) (end 192.023 57.15) (width 0.5) (layer "F.Cu") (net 4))
 (segment (start 176.53 59.437) (end 174.243 57.15) (width 0.5) (layer "F.Cu") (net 4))
 (segment (start 174.243 57.15) (end 176.53 54.863) (width 0.5) (layer "F.Cu") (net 4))
 (segment (start 165.84875 84.6825) (end 163.98625 82.82) (width 0.5) (layer "F.Cu") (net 4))
 (segment (start 157.4125 79.715) (end 157.1175 80.01) (width 0.5) (layer "F.Cu") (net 4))
 (segment (start 153.67 68.58) (end 153.67 67.31) (width 0.5) (layer "F.Cu") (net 4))
 (segment (start 141.605 55.49) (end 141.605 58.42) (width 0.5) (layer "F.Cu") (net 4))
 (segment (start 174.243 69.85) (end 176.53 67.563) (width 0.5) (layer "F.Cu") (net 4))
 (segment (start 194.31 80.263) (end 192.023 82.55) (width 0.5) (layer "F.Cu") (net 4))
 (segment (start 158.75 81.6425) (end 157.1175 80.01) (width 0.25) (layer "F.Cu") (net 4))
 (segment (start 192.023 69.85) (end 194.31 72.137) (width 0.5) (layer "F.Cu") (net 4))
 (segment (start 180.34 88.265) (end 179.07 89.535) (width 0.5) (layer "F.Cu") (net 4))
 (segment (start 158.75 82.82) (end 162.56 82.82) (width 0.25) (layer "F.Cu") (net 4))
 (segment (start 157.4125 78.105) (end 157.4125 79.715) (width 0.5) (layer "F.Cu") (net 4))
 (segment (start 172.973 81.28) (end 174.243 82.55) (width 0.5) (layer "F.Cu") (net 4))
 (segment (start 189.738 54.865) (end 189.738 46.735) (width 0.5) (layer "F.Cu") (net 4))
 (segment (start 171.7635 81.28) (end 172.973 81.28) (width 0.5) (layer "F.Cu") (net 4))
 (segment (start 138.185 52.07) (end 141.605 55.49) (width 0.5) (layer "F.Cu") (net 4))
 (segment (start 176.53 54.863) (end 176.53 46.737) (width 0.5) (layer "F.Cu") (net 4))
 (segment (start 158.75 82.82) (end 158.75 81.6425) (width 0.25) (layer "F.Cu") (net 4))
 (segment (start 174.243 82.55) (end 177.8 82.55) (width 0.5) (layer "F.Cu") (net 4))
 (segment (start 176.53 67.563) (end 176.53 59.437) (width 0.5) (layer "F.Cu") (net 4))
 (segment (start 180.34 71.12) (end 180.34 80.01) (width 0.5) (layer "F.Cu") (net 4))
 (segment (start 180.34 80.01) (end 180.34 88.265) (width 0.5) (layer "F.Cu") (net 4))
 (segment (start 179.07 69.85) (end 192.023 69.85) (width 0.5) (layer "F.Cu") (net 4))
 (segment (start 174.243 77.47) (end 161.925 77.47) (width 0.5) (layer "F.Cu") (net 1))
 (segment (start 155.6875 77.3575) (end 155.6875 78.105) (width 0.5) (layer "F.Cu") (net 1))
 (segment (start 161.925 77.47) (end 160.655 76.2) (width 0.5) (layer "F.Cu") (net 1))
 (segment (start 146.05 83.185) (end 154.305 74.93) (width 0.5) (layer "F.Cu") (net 1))
 (segment (start 156.845 76.2) (end 155.6875 77.3575) (width 0.5) (layer "F.Cu") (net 1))
 (segment (start 154.35 81.6425) (end 155.9825 80.01) (width 0.25) (layer "F.Cu") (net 1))
 (segment (start 135.255 83.185) (end 145.415 83.185) (width 0.5) (layer "F.Cu") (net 1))
 (segment (start 154.94 74.93) (end 155.575 74.93) (width 0.5) (layer "F.Cu") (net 1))
 (segment (start 155.6875 78.105) (end 155.6875 79.715) (width 0.5) (layer "F.Cu") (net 1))
 (segment (start 148.59 74.93) (end 154.94 74.93) (width 0.5) (layer "F.Cu") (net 1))
 (segment (start 155.6875 79.715) (end 155.9825 80.01) (width 0.5) (layer "F.Cu") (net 1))
 (segment (start 154.305 74.93) (end 154.94 74.93) (width 0.5) (layer "F.Cu") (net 1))
 (segment (start 154.35 82.82) (end 154.35 81.6425) (width 0.25) (layer "F.Cu") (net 1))
 (segment (start 145.415 83.185) (end 146.05 83.185) (width 0.5) (layer "F.Cu") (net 1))
 (segment (start 160.655 76.2) (end 156.845 76.2) (width 0.5) (layer "F.Cu") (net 1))
 (segment (start 155.575 74.93) (end 156.845 76.2) (width 0.5) (layer "F.Cu") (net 1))
 (via (at 148.59 74.93) (size 0.8) (drill 0.4) (layers "F.Cu" "B.Cu") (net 1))
 (segment (start 148.59 68.58) (end 148.59 74.93) (width 0.5) (layer "B.Cu") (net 1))
 (segment (start 166.37 82.9575) (end 169.418 82.9575) (width 0.5) (layer "F.Cu") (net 3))
 (segment (start 166.37 82.9575) (end 167.2325 82.9575) (width 0.5) (layer "F.Cu") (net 3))
 (segment (start 171.45 82.9575) (end 170.6285 82.136) (width 0.5) (layer "F.Cu") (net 3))
 (segment (start 171.45 82.9575) (end 172.1105 82.9575) (width 0.5) (layer "F.Cu") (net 3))
 (segment (start 169.418 82.9575) (end 171.45 82.9575) (width 0.5) (layer "F.Cu") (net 3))
 (segment (start 172.1105 82.9575) (end 174.243 85.09) (width 0.5) (layer "F.Cu") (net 3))
 (segment (start 167.2325 82.9575) (end 168.91 81.28) (width 0.5) (layer "F.Cu") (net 3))
 (segment (start 170.6285 82.136) (end 170.6285 81.28) (width 0.5) (layer "F.Cu") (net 3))
 (via (at 168.91 81.28) (size 0.8) (drill 0.4) (layers "F.Cu" "B.Cu") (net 3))
 (segment (start 170.815 55.88) (end 163.83 48.895) (width 0.5) (layer "B.Cu") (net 3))
 (segment (start 137.16 48.895) (end 133.985 52.07) (width 0.5) (layer "B.Cu") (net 3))
 (segment (start 163.83 48.895) (end 137.16 48.895) (width 0.5) (layer "B.Cu") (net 3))
 (segment (start 170.815 79.375) (end 170.815 55.88) (width 0.5) (layer "B.Cu") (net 3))
 (segment (start 168.91 81.28) (end 170.815 79.375) (width 0.5) (layer "B.Cu") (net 3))
 (segment (start 158.75 84.82) (end 162.195 84.82) (width 0.25) (layer "F.Cu") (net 39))
 (segment (start 162.195 84.82) (end 163.195 83.82) (width 0.25) (layer "F.Cu") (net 39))
 (via (at 163.195 83.82) (size 0.8) (drill 0.4) (layers "F.Cu" "B.Cu") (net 39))
 (segment (start 144.78 60.96) (end 163.195 60.96) (width 0.25) (layer "B.Cu") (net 39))
 (segment (start 136.691 54.864) (end 138.684 54.864) (width 0.25) (layer "B.Cu") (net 39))
 (segment (start 169.545 67.31) (end 169.545 77.47) (width 0.25) (layer "B.Cu") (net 39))
 (segment (start 169.545 77.47) (end 163.195 83.82) (width 0.25) (layer "B.Cu") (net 39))
 (segment (start 133.985 57.57) (end 136.691 54.864) (width 0.25) (layer "B.Cu") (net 39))
 (segment (start 138.684 54.864) (end 144.78 60.96) (width 0.25) (layer "B.Cu") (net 39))
 (segment (start 163.195 60.96) (end 169.545 67.31) (width 0.25) (layer "B.Cu") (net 39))
 (segment (start 160.79 84.32) (end 161.29 83.82) (width 0.25) (layer "F.Cu") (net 40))
 (segment (start 158.75 84.32) (end 160.79 84.32) (width 0.25) (layer "F.Cu") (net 40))
 (via (at 161.29 83.82) (size 0.8) (drill 0.4) (layers "F.Cu" "B.Cu") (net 40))
 (segment (start 162.56 62.23) (end 168.275 67.945) (width 0.25) (layer "B.Cu") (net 40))
 (segment (start 142.845 62.23) (end 162.56 62.23) (width 0.25) (layer "B.Cu") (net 40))
 (segment (start 168.275 76.835) (end 161.29 83.82) (width 0.25) (layer "B.Cu") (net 40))
 (segment (start 168.275 67.945) (end 168.275 76.835) (width 0.25) (layer "B.Cu") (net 40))
 (segment (start 138.185 57.57) (end 142.845 62.23) (width 0.25) (layer "B.Cu") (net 40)))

